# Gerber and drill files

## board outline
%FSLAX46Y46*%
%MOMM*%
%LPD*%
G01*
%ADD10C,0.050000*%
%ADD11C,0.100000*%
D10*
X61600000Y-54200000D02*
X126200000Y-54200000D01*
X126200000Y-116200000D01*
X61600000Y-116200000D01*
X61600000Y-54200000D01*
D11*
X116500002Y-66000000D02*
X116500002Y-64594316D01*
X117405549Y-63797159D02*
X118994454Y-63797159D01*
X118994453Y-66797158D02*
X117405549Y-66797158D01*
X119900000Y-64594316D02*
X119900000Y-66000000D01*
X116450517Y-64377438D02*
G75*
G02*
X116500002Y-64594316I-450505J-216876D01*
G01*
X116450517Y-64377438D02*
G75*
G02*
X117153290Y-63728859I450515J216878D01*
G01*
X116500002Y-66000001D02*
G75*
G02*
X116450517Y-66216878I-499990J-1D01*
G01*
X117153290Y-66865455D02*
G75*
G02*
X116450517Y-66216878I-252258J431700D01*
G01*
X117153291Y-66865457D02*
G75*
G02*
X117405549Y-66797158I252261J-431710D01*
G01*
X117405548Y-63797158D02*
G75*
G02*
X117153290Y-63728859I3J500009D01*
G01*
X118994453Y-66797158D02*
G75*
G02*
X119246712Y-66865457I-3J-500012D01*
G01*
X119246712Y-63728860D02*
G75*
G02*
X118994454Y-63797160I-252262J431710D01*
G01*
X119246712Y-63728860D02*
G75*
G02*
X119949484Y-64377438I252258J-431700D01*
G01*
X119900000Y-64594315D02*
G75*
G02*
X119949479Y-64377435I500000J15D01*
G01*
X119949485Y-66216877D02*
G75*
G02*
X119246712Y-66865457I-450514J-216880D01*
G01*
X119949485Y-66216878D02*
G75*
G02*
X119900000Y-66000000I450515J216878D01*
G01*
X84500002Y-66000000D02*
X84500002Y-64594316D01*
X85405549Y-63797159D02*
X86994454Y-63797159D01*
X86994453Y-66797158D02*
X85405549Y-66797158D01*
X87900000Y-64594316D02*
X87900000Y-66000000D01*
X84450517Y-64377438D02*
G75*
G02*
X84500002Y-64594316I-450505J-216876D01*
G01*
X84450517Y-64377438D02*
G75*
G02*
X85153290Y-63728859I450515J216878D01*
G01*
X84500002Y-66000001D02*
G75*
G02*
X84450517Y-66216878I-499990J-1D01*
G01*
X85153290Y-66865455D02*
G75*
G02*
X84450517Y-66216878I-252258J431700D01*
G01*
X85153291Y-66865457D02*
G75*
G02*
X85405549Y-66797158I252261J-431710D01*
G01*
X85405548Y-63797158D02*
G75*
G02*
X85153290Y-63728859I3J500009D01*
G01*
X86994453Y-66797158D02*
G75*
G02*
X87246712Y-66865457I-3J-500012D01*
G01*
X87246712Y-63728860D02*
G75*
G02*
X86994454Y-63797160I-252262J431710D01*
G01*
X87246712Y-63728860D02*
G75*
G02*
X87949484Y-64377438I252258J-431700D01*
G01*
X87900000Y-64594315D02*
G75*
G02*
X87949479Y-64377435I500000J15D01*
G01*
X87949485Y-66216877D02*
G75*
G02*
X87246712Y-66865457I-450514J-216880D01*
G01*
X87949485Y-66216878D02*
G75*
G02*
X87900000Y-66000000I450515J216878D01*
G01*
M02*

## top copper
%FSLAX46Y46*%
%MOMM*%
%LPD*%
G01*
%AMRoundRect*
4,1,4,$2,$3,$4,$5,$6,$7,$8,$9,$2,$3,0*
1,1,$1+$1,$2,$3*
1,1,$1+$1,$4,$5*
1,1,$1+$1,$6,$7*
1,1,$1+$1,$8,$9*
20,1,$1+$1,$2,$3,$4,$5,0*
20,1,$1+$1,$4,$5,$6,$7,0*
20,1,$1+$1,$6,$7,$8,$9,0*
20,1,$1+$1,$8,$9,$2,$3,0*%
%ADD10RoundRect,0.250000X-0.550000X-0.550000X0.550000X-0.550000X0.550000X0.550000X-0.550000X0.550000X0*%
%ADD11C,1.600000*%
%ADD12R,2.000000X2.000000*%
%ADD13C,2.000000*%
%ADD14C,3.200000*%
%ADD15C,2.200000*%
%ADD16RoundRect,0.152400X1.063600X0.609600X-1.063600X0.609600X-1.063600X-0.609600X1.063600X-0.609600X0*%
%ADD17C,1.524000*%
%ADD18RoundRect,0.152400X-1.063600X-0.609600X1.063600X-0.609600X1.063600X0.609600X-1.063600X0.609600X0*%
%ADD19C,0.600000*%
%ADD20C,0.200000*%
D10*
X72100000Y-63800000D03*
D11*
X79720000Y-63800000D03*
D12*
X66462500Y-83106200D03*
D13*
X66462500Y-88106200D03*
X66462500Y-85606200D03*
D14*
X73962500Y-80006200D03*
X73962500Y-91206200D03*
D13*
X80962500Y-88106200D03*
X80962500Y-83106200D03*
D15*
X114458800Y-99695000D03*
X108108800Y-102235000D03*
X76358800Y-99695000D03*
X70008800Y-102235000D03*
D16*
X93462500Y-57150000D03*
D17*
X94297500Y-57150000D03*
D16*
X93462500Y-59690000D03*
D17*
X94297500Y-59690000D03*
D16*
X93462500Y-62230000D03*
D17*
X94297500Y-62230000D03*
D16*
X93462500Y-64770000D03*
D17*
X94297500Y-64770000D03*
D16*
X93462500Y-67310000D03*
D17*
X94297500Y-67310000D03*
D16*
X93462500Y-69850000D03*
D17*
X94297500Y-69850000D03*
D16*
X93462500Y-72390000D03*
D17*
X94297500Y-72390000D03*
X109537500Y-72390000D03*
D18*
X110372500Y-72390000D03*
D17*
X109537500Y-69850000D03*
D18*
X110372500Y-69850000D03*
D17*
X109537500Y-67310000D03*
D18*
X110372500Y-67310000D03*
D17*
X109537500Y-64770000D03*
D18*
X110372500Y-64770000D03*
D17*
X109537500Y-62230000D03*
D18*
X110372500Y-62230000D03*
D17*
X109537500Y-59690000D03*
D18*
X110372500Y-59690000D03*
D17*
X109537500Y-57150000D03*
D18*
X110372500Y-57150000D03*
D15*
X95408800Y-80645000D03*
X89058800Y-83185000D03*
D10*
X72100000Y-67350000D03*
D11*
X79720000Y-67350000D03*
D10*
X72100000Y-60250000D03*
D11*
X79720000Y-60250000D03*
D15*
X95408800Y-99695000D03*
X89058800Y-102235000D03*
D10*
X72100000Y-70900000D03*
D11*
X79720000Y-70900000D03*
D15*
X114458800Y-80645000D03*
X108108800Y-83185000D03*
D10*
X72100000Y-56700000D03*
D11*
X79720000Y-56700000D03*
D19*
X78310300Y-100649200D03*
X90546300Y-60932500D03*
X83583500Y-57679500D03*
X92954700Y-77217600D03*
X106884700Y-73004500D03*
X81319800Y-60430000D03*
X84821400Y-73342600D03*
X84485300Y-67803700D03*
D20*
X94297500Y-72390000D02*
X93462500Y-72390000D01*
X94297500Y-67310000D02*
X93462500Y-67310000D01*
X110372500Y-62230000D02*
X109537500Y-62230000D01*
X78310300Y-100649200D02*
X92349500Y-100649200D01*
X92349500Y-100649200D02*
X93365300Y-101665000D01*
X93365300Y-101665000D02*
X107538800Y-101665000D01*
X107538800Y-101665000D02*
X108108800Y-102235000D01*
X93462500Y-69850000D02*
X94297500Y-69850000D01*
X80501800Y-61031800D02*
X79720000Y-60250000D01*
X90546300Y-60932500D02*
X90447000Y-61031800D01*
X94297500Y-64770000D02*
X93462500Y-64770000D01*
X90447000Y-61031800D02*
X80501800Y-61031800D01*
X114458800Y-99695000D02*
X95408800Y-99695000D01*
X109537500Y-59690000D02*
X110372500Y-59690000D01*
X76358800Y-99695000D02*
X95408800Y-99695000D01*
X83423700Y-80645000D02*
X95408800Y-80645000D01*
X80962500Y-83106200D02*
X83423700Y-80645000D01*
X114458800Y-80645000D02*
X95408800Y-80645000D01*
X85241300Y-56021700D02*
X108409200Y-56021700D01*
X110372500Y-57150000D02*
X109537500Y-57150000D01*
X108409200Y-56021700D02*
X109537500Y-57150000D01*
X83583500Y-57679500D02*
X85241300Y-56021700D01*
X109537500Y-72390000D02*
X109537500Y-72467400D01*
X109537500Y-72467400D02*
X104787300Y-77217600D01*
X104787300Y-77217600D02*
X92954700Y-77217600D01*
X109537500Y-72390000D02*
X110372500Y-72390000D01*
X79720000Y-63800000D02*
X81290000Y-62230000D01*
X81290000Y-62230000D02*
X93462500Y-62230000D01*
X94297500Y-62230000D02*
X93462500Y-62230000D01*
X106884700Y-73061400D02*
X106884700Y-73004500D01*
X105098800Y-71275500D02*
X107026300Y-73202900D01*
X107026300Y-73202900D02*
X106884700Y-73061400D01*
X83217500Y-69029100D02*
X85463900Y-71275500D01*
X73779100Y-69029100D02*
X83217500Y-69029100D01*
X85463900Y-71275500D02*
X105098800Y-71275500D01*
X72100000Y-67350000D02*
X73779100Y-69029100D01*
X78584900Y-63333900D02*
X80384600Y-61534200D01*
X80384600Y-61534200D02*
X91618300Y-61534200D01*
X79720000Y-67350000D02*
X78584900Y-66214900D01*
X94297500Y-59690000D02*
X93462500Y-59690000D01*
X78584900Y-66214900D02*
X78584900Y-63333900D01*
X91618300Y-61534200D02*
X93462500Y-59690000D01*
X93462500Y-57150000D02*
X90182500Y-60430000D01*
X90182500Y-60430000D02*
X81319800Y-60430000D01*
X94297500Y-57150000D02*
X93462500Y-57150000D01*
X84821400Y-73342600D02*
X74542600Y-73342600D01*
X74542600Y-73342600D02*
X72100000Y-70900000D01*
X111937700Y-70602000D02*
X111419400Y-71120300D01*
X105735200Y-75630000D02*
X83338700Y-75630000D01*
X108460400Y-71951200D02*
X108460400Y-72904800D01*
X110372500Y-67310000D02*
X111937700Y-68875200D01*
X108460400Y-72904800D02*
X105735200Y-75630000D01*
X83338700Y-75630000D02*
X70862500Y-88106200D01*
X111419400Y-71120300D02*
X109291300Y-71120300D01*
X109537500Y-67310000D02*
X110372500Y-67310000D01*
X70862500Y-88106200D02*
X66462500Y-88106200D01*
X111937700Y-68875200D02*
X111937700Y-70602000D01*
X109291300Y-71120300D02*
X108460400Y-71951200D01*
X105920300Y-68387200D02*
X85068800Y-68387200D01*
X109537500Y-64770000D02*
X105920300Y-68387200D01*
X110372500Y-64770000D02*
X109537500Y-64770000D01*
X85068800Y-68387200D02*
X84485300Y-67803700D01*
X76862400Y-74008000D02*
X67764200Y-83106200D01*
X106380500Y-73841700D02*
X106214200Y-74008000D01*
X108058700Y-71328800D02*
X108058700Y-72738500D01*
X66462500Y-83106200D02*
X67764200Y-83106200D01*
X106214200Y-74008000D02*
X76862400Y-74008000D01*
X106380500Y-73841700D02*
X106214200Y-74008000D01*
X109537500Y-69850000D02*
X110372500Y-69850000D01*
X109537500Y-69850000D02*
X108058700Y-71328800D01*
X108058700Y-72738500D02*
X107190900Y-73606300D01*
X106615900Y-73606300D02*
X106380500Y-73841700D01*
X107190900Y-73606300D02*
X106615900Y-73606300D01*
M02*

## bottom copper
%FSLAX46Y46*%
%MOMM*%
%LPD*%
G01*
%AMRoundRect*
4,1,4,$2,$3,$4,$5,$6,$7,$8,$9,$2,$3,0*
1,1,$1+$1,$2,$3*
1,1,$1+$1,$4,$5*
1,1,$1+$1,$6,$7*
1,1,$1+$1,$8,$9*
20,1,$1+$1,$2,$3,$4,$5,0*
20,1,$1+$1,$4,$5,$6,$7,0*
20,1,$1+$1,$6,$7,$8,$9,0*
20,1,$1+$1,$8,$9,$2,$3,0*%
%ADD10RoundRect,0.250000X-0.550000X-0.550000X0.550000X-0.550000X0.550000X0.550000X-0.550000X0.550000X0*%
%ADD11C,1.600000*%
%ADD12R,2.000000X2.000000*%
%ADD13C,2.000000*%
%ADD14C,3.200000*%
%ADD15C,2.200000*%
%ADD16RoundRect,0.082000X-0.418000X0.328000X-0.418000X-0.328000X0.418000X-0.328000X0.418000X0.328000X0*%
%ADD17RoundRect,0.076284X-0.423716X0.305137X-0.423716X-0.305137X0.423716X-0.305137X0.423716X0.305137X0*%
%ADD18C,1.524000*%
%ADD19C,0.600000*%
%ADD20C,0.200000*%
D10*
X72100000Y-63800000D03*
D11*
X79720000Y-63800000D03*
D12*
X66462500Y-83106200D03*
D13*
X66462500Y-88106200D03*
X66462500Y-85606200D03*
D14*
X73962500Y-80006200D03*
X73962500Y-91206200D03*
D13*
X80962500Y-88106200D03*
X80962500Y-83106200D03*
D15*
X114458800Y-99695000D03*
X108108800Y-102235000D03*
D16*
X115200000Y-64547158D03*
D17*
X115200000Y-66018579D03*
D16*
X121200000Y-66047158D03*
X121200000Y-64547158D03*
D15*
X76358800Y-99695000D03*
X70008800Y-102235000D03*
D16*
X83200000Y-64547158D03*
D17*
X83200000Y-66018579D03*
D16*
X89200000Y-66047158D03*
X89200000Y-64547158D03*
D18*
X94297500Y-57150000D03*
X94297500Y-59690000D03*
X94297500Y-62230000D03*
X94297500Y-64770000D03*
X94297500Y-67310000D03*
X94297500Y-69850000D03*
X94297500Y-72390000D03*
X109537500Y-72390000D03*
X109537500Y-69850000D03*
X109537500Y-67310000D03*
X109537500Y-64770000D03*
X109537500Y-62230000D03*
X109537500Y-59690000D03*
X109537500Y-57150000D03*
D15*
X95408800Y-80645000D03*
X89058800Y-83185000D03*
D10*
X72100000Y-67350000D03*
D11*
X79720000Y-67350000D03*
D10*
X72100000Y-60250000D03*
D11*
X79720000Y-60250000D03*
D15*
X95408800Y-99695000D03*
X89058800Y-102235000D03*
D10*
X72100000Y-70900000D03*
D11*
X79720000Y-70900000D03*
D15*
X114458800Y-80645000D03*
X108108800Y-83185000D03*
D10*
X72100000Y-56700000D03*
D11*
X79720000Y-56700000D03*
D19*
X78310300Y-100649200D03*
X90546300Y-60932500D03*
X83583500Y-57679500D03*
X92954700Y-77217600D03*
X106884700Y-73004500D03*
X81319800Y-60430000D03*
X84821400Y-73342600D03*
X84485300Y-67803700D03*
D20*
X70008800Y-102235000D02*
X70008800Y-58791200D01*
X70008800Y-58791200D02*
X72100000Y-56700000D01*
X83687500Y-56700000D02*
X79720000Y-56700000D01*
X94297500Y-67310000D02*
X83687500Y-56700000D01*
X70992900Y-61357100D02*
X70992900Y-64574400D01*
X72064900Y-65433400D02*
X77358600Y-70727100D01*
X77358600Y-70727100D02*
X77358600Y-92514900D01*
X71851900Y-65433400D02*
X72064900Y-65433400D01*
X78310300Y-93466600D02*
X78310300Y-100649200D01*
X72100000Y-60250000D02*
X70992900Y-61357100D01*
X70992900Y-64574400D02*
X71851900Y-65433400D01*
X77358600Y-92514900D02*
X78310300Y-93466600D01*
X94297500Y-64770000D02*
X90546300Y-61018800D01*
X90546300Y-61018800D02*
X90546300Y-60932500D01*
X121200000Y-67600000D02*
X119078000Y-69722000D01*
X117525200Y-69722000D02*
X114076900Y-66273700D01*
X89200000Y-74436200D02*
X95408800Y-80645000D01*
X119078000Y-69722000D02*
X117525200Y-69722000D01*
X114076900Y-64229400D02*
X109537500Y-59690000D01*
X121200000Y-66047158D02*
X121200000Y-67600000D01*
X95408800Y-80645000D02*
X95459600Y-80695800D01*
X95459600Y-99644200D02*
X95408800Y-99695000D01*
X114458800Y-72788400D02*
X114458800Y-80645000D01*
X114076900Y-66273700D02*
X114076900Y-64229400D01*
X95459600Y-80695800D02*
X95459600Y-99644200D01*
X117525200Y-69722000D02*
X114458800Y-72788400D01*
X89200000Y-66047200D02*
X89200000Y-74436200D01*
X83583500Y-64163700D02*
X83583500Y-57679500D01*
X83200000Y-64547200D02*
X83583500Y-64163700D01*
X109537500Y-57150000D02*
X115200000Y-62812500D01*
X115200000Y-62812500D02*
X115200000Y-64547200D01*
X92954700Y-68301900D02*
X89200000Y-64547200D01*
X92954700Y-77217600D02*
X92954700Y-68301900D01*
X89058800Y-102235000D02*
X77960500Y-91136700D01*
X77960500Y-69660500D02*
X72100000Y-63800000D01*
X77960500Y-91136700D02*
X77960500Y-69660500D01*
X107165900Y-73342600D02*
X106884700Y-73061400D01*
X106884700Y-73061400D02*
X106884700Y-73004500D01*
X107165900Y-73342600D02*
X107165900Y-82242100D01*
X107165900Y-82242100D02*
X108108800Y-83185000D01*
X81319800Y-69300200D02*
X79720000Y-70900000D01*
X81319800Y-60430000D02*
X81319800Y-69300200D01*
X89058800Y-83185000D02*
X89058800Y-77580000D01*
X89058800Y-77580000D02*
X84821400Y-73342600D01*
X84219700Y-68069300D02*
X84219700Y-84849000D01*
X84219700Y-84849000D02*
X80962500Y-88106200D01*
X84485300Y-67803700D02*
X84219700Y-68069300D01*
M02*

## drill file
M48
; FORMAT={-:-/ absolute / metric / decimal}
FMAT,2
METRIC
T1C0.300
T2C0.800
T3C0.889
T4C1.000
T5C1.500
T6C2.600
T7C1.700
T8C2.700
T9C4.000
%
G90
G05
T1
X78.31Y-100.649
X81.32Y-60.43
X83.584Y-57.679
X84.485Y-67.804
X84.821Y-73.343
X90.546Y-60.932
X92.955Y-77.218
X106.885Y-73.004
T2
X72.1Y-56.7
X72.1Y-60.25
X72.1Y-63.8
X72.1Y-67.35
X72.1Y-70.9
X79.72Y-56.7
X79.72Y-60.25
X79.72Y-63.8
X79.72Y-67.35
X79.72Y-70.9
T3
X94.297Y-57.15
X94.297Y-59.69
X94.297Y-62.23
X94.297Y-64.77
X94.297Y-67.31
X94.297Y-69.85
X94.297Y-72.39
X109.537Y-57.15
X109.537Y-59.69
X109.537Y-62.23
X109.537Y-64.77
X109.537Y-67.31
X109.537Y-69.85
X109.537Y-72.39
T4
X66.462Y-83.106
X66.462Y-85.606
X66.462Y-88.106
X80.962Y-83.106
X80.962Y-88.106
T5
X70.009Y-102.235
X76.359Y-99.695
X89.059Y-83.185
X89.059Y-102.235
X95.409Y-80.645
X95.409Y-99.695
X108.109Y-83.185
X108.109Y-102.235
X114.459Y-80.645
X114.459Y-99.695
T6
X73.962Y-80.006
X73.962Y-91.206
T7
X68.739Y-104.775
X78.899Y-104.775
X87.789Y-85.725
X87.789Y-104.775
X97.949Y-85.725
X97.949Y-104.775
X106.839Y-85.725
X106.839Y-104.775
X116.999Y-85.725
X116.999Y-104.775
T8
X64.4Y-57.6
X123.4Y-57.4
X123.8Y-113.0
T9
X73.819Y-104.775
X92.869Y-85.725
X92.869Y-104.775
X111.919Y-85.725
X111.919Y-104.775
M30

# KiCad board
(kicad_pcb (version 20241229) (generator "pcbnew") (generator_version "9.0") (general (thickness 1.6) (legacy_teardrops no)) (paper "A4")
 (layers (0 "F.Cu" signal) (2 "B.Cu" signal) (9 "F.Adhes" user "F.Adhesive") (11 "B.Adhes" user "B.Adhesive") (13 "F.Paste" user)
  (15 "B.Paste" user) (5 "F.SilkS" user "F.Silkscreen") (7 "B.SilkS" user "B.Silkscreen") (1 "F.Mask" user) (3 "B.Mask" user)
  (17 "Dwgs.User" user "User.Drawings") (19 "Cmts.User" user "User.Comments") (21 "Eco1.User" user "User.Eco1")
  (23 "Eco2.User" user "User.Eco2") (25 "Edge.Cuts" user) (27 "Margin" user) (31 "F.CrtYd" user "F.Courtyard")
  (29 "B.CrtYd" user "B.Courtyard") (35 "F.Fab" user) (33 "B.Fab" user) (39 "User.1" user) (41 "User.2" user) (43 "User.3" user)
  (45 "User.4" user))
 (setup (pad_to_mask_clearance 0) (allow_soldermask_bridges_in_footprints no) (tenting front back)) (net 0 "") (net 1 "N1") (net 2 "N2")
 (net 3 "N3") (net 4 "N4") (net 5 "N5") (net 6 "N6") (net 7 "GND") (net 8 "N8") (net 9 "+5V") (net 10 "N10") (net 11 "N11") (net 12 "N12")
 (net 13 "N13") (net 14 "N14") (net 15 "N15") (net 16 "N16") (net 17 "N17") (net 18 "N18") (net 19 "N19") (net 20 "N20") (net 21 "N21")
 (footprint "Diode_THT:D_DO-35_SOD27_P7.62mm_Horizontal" (layer "F.Cu") (at 72.1 63.8)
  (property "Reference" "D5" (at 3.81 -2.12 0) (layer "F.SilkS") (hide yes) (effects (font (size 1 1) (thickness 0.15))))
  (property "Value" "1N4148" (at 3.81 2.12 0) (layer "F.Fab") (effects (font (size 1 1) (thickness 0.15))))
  (pad "1" thru_hole roundrect (at 0 0) (size 1.6 1.6) (drill 0.8) (layers "*.Cu" "*.Mask") (remove_unused_layers no)
   (roundrect_rratio 0.15625) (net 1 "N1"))
  (pad "2" thru_hole circle (at 7.62 0) (size 1.6 1.6) (drill 0.8) (layers "*.Cu" "*.Mask") (remove_unused_layers no) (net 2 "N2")))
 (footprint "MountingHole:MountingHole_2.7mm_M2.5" (layer "F.Cu") (at 123.4 57.4)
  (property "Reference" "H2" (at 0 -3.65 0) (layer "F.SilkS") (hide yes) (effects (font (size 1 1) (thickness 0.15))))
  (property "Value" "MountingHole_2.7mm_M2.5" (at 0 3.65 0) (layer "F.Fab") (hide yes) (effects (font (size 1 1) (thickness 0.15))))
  (pad "" np_thru_hole circle (at 0 0) (size 2.7 2.7) (drill 2.7) (layers "*.Cu" "*.Mask")))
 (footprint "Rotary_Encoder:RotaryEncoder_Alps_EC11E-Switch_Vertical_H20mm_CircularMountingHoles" (layer "F.Cu") (at 66.4625 83.1062)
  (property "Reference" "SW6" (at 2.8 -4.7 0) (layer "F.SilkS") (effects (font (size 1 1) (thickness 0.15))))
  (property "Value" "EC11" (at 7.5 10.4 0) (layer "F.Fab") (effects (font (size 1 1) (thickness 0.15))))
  (pad "A" thru_hole rect (at 0 0) (size 2 2) (drill 1) (layers "*.Cu" "*.Mask") (remove_unused_layers no) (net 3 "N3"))
  (pad "B" thru_hole circle (at 0 5) (size 2 2) (drill 1) (layers "*.Cu" "*.Mask") (remove_unused_layers no) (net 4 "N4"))
  (pad "C" thru_hole circle (at 0 2.5) (size 2 2) (drill 1) (layers "*.Cu" "*.Mask") (remove_unused_layers no) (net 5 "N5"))
  (pad "MP" thru_hole circle (at 7.5 -3.1) (size 3.2 3.2) (drill 2.6) (layers "*.Cu" "*.Mask") (remove_unused_layers no))
  (pad "MP" thru_hole circle (at 7.5 8.1) (size 3.2 3.2) (drill 2.6) (layers "*.Cu" "*.Mask") (remove_unused_layers no))
  (pad "S1" thru_hole circle (at 14.5 5) (size 2 2) (drill 1) (layers "*.Cu" "*.Mask") (remove_unused_layers no) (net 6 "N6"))
  (pad "S2" thru_hole circle (at 14.5 0) (size 2 2) (drill 1) (layers "*.Cu" "*.Mask") (remove_unused_layers no) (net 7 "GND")))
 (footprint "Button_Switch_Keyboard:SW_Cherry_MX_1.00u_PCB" (layer "F.Cu") (at 114.4588 99.695)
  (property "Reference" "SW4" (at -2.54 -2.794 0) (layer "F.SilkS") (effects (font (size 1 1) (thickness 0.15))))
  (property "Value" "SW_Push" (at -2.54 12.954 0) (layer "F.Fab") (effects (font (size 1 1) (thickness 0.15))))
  (pad "" np_thru_hole circle (at -7.62 5.08) (size 1.7 1.7) (drill 1.7) (layers "*.Cu" "*.Mask"))
  (pad "" np_thru_hole circle (at -2.54 5.08) (size 4 4) (drill 4) (layers "*.Cu" "*.Mask"))
  (pad "" np_thru_hole circle (at 2.54 5.08) (size 1.7 1.7) (drill 1.7) (layers "*.Cu" "*.Mask"))
  (pad "1" thru_hole circle (at 0 0) (size 2.2 2.2) (drill 1.5) (layers "*.Cu" "*.Mask") (remove_unused_layers no) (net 7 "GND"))
  (pad "2" thru_hole circle (at -6.35 2.54) (size 2.2 2.2) (drill 1.5) (layers "*.Cu" "*.Mask") (remove_unused_layers no) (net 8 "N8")))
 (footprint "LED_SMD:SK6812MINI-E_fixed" (layer "F.Cu") (at 118.2 65.4)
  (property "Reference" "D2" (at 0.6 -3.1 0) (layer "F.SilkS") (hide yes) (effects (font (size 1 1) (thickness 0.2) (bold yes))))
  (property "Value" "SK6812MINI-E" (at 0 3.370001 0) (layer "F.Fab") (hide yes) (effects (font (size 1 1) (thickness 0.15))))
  (fp_line (start -1.699998 0.6) (end -1.699998 -0.805684) (stroke (width 0.1) (type solid)) (layer "Edge.Cuts"))
  (fp_line (start -0.794451 -1.602841) (end 0.794454 -1.602841) (stroke (width 0.1) (type solid)) (layer "Edge.Cuts"))
  (fp_line (start 0.794453 1.397158) (end -0.794451 1.397158) (stroke (width 0.1) (type solid)) (layer "Edge.Cuts"))
  (fp_line (start 1.7 -0.805684) (end 1.7 0.6) (stroke (width 0.1) (type solid)) (layer "Edge.Cuts"))
  (fp_arc (start -1.749483 -1.022562) (mid -1.712526 -0.91691) (end -1.699998 -0.805684) (stroke (width 0.1) (type solid))
   (layer "Edge.Cuts"))
  (fp_arc (start -1.749483 -1.022562) (mid -1.63807 -1.606877) (end -1.04671 -1.671141) (stroke (width 0.1) (type solid))
   (layer "Edge.Cuts"))
  (fp_arc (start -1.699998 0.600001) (mid -1.712526 0.711226) (end -1.749483 0.816878) (stroke (width 0.1) (type solid)) (layer "Edge.Cuts"))
  (fp_arc (start -1.04671 1.465455) (mid -1.638069 1.401192) (end -1.749483 0.816878) (stroke (width 0.1) (type solid)) (layer "Edge.Cuts"))
  (fp_arc (start -1.046709 1.465457) (mid -0.925121 1.414535) (end -0.794451 1.397158) (stroke (width 0.1) (type solid)) (layer "Edge.Cuts"))
  (fp_arc (start -0.794452 -1.602842) (mid -0.925122 -1.620219) (end -1.04671 -1.671141) (stroke (width 0.1) (type solid))
   (layer "Edge.Cuts"))
  (fp_arc (start 0.794453 1.397158) (mid 0.925124 1.414535) (end 1.046712 1.465457) (stroke (width 0.1) (type solid)) (layer "Edge.Cuts"))
  (fp_arc (start 1.046712 -1.67114) (mid 0.925124 -1.620218) (end 0.794454 -1.602841) (stroke (width 0.1) (type solid)) (layer "Edge.Cuts"))
  (fp_arc (start 1.046712 -1.67114) (mid 1.638072 -1.606876) (end 1.749485 -1.022562) (stroke (width 0.1) (type solid)) (layer "Edge.Cuts"))
  (fp_arc (start 1.7 -0.805685) (mid 1.712528 -0.91691) (end 1.749485 -1.022562) (stroke (width 0.1) (type solid)) (layer "Edge.Cuts"))
  (fp_arc (start 1.749485 0.816877) (mid 1.638073 1.401193) (end 1.046712 1.465457) (stroke (width 0.1) (type solid)) (layer "Edge.Cuts"))
  (fp_arc (start 1.749485 0.816878) (mid 1.712528 0.711226) (end 1.7 0.6) (stroke (width 0.1) (type solid)) (layer "Edge.Cuts"))
  (pad "1" smd roundrect (at -3 -0.852842 270) (size 0.82 1) (layers "B.Cu" "B.Mask" "B.Paste") (roundrect_rratio 0.1) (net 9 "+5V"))
  (pad "2" smd roundrect (at -3 0.618579 270) (size 0.762842 1) (layers "B.Cu" "B.Mask" "B.Paste") (roundrect_rratio 0.1))
  (pad "3" smd roundrect (at 3 0.647158 270) (size 0.82 1) (layers "B.Cu" "B.Mask" "B.Paste") (roundrect_rratio 0.1) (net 7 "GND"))
  (pad "4" smd roundrect (at 3 -0.852842 270) (size 0.82 1) (layers "B.Cu" "B.Mask" "B.Paste") (roundrect_rratio 0.1) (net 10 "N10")))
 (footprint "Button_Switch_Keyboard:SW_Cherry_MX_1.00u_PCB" (layer "F.Cu") (at 76.3588 99.695)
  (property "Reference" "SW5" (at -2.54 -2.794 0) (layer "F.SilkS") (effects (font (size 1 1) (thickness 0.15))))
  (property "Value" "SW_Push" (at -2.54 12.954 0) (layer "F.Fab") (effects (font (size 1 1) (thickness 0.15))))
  (pad "" np_thru_hole circle (at -7.62 5.08) (size 1.7 1.7) (drill 1.7) (layers "*.Cu" "*.Mask"))
  (pad "" np_thru_hole circle (at -2.54 5.08) (size 4 4) (drill 4) (layers "*.Cu" "*.Mask"))
  (pad "" np_thru_hole circle (at 2.54 5.08) (size 1.7 1.7) (drill 1.7) (layers "*.Cu" "*.Mask"))
  (pad "1" thru_hole circle (at 0 0) (size 2.2 2.2) (drill 1.5) (layers "*.Cu" "*.Mask") (remove_unused_layers no) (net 7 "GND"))
  (pad "2" thru_hole circle (at -6.35 2.54) (size 2.2 2.2) (drill 1.5) (layers "*.Cu" "*.Mask") (remove_unused_layers no) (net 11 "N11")))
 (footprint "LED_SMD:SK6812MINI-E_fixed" (layer "F.Cu") (at 86.2 65.4)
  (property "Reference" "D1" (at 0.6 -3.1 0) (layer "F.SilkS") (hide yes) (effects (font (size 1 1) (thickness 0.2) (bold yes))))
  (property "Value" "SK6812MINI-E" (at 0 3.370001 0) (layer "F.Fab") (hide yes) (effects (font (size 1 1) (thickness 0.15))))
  (fp_line (start -1.699998 0.6) (end -1.699998 -0.805684) (stroke (width 0.1) (type solid)) (layer "Edge.Cuts"))
  (fp_line (start -0.794451 -1.602841) (end 0.794454 -1.602841) (stroke (width 0.1) (type solid)) (layer "Edge.Cuts"))
  (fp_line (start 0.794453 1.397158) (end -0.794451 1.397158) (stroke (width 0.1) (type solid)) (layer "Edge.Cuts"))
  (fp_line (start 1.7 -0.805684) (end 1.7 0.6) (stroke (width 0.1) (type solid)) (layer "Edge.Cuts"))
  (fp_arc (start -1.749483 -1.022562) (mid -1.712526 -0.91691) (end -1.699998 -0.805684) (stroke (width 0.1) (type solid))
   (layer "Edge.Cuts"))
  (fp_arc (start -1.749483 -1.022562) (mid -1.63807 -1.606877) (end -1.04671 -1.671141) (stroke (width 0.1) (type solid))
   (layer "Edge.Cuts"))
  (fp_arc (start -1.699998 0.600001) (mid -1.712526 0.711226) (end -1.749483 0.816878) (stroke (width 0.1) (type solid)) (layer "Edge.Cuts"))
  (fp_arc (start -1.04671 1.465455) (mid -1.638069 1.401192) (end -1.749483 0.816878) (stroke (width 0.1) (type solid)) (layer "Edge.Cuts"))
  (fp_arc (start -1.046709 1.465457) (mid -0.925121 1.414535) (end -0.794451 1.397158) (stroke (width 0.1) (type solid)) (layer "Edge.Cuts"))
  (fp_arc (start -0.794452 -1.602842) (mid -0.925122 -1.620219) (end -1.04671 -1.671141) (stroke (width 0.1) (type solid))
   (layer "Edge.Cuts"))
  (fp_arc (start 0.794453 1.397158) (mid 0.925124 1.414535) (end 1.046712 1.465457) (stroke (width 0.1) (type solid)) (layer "Edge.Cuts"))
  (fp_arc (start 1.046712 -1.67114) (mid 0.925124 -1.620218) (end 0.794454 -1.602841) (stroke (width 0.1) (type solid)) (layer "Edge.Cuts"))
  (fp_arc (start 1.046712 -1.67114) (mid 1.638072 -1.606876) (end 1.749485 -1.022562) (stroke (width 0.1) (type solid)) (layer "Edge.Cuts"))
  (fp_arc (start 1.7 -0.805685) (mid 1.712528 -0.91691) (end 1.749485 -1.022562) (stroke (width 0.1) (type solid)) (layer "Edge.Cuts"))
  (fp_arc (start 1.749485 0.816877) (mid 1.638073 1.401193) (end 1.046712 1.465457) (stroke (width 0.1) (type solid)) (layer "Edge.Cuts"))
  (fp_arc (start 1.749485 0.816878) (mid 1.712528 0.711226) (end 1.7 0.6) (stroke (width 0.1) (type solid)) (layer "Edge.Cuts"))
  (pad "1" smd roundrect (at -3 -0.852842 270) (size 0.82 1) (layers "B.Cu" "B.Mask" "B.Paste") (roundrect_rratio 0.1) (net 9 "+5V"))
  (pad "2" smd roundrect (at -3 0.618579 270) (size 0.762842 1) (layers "B.Cu" "B.Mask" "B.Paste") (roundrect_rratio 0.1))
  (pad "3" smd roundrect (at 3 0.647158 270) (size 0.82 1) (layers "B.Cu" "B.Mask" "B.Paste") (roundrect_rratio 0.1) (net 7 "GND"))
  (pad "4" smd roundrect (at 3 -0.852842 270) (size 0.82 1) (layers "B.Cu" "B.Mask" "B.Paste") (roundrect_rratio 0.1) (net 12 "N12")))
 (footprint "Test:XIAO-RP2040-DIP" (layer "F.Cu") (at 101.9175 64.77)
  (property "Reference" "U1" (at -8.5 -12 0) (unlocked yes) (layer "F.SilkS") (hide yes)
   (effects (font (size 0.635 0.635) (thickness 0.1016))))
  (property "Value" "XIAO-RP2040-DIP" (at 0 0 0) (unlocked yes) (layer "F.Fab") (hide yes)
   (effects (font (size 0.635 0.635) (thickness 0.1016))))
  (pad "1" smd roundrect (at -8.455 -7.62 180) (size 2.432 1.524) (layers "F.Cu" "F.Mask") (roundrect_rratio 0.1) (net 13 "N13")
   (thermal_bridge_angle 45))
  (pad "1" thru_hole circle (at -7.62 -7.62 180) (size 1.524 1.524) (drill 0.889) (layers "*.Cu" "*.Mask") (remove_unused_layers no)
   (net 13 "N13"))
  (pad "2" smd roundrect (at -8.455 -5.08 180) (size 2.432 1.524) (layers "F.Cu" "F.Mask") (roundrect_rratio 0.1) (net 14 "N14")
   (thermal_bridge_angle 45))
  (pad "2" thru_hole circle (at -7.62 -5.08 180) (size 1.524 1.524) (drill 0.889) (layers "*.Cu" "*.Mask") (remove_unused_layers no)
   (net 14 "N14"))
  (pad "3" smd roundrect (at -8.455 -2.54 180) (size 2.432 1.524) (layers "F.Cu" "F.Mask") (roundrect_rratio 0.1) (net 2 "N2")
   (thermal_bridge_angle 45))
  (pad "3" thru_hole circle (at -7.62 -2.54 180) (size 1.524 1.524) (drill 0.889) (layers "*.Cu" "*.Mask") (remove_unused_layers no)
   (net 2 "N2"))
  (pad "4" smd roundrect (at -8.455 0 180) (size 2.432 1.524) (layers "F.Cu" "F.Mask") (roundrect_rratio 0.1) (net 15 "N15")
   (thermal_bridge_angle 45))
  (pad "4" thru_hole circle (at -7.62 0 180) (size 1.524 1.524) (drill 0.889) (layers "*.Cu" "*.Mask") (remove_unused_layers no)
   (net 15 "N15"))
  (pad "5" smd roundrect (at -8.455 2.54 180) (size 2.432 1.524) (layers "F.Cu" "F.Mask") (roundrect_rratio 0.1) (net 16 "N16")
   (thermal_bridge_angle 45))
  (pad "5" thru_hole circle (at -7.62 2.54 180) (size 1.524 1.524) (drill 0.889) (layers "*.Cu" "*.Mask") (remove_unused_layers no)
   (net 16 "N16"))
  (pad "6" smd roundrect (at -8.455 5.08 180) (size 2.432 1.524) (layers "F.Cu" "F.Mask") (roundrect_rratio 0.1) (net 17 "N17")
   (thermal_bridge_angle 45))
  (pad "6" thru_hole circle (at -7.62 5.08 180) (size 1.524 1.524) (drill 0.889) (layers "*.Cu" "*.Mask") (remove_unused_layers no)
   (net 17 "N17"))
  (pad "7" smd roundrect (at -8.455 7.62 180) (size 2.432 1.524) (layers "F.Cu" "F.Mask") (roundrect_rratio 0.1) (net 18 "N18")
   (thermal_bridge_angle 45))
  (pad "7" thru_hole circle (at -7.62 7.62 180) (size 1.524 1.524) (drill 0.889) (layers "*.Cu" "*.Mask") (remove_unused_layers no)
   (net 18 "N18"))
  (pad "8" thru_hole circle (at 7.62 7.62) (size 1.524 1.524) (drill 0.889) (layers "*.Cu" "*.Mask") (remove_unused_layers no)
   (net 12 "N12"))
  (pad "8" smd roundrect (at 8.455 7.62) (size 2.432 1.524) (layers "F.Cu" "F.Mask") (roundrect_rratio 0.1) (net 12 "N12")
   (thermal_bridge_angle 45))
  (pad "9" thru_hole circle (at 7.62 5.08) (size 1.524 1.524) (drill 0.889) (layers "*.Cu" "*.Mask") (remove_unused_layers no) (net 3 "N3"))
  (pad "9" smd roundrect (at 8.455 5.08) (size 2.432 1.524) (layers "F.Cu" "F.Mask") (roundrect_rratio 0.1) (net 3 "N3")
   (thermal_bridge_angle 45))
  (pad "10" thru_hole circle (at 7.62 2.54) (size 1.524 1.524) (drill 0.889) (layers "*.Cu" "*.Mask") (remove_unused_layers no) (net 4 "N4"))
  (pad "10" smd roundrect (at 8.455 2.54) (size 2.432 1.524) (layers "F.Cu" "F.Mask") (roundrect_rratio 0.1) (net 4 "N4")
   (thermal_bridge_angle 45))
  (pad "11" thru_hole circle (at 7.62 0) (size 1.524 1.524) (drill 0.889) (layers "*.Cu" "*.Mask") (remove_unused_layers no) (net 6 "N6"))
  (pad "11" smd roundrect (at 8.455 0) (size 2.432 1.524) (layers "F.Cu" "F.Mask") (roundrect_rratio 0.1) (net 6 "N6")
   (thermal_bridge_angle 45))
  (pad "12" thru_hole circle (at 7.62 -2.54) (size 1.524 1.524) (drill 0.889) (layers "*.Cu" "*.Mask") (remove_unused_layers no)
   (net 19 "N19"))
  (pad "12" smd roundrect (at 8.455 -2.54) (size 2.432 1.524) (layers "F.Cu" "F.Mask") (roundrect_rratio 0.1) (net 19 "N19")
   (thermal_bridge_angle 45))
  (pad "13" thru_hole circle (at 7.62 -5.08) (size 1.524 1.524) (drill 0.889) (layers "*.Cu" "*.Mask") (remove_unused_layers no)
   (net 7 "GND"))
  (pad "13" smd roundrect (at 8.455 -5.08) (size 2.432 1.524) (layers "F.Cu" "F.Mask") (roundrect_rratio 0.1) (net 7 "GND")
   (thermal_bridge_angle 45))
  (pad "14" thru_hole circle (at 7.62 -7.62) (size 1.524 1.524) (drill 0.889) (layers "*.Cu" "*.Mask") (remove_unused_layers no)
   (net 9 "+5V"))
  (pad "14" smd roundrect (at 8.455 -7.62) (size 2.432 1.524) (layers "F.Cu" "F.Mask") (roundrect_rratio 0.1) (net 9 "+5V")
   (thermal_bridge_angle 45)))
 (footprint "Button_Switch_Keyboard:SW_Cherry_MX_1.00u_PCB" (layer "F.Cu") (at 95.4088 80.645)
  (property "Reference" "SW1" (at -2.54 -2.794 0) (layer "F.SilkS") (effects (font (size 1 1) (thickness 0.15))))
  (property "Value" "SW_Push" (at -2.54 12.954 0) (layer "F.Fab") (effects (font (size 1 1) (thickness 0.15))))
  (pad "" np_thru_hole circle (at -7.62 5.08) (size 1.7 1.7) (drill 1.7) (layers "*.Cu" "*.Mask"))
  (pad "" np_thru_hole circle (at -2.54 5.08) (size 4 4) (drill 4) (layers "*.Cu" "*.Mask"))
  (pad "" np_thru_hole circle (at 2.54 5.08) (size 1.7 1.7) (drill 1.7) (layers "*.Cu" "*.Mask"))
  (pad "1" thru_hole circle (at 0 0) (size 2.2 2.2) (drill 1.5) (layers "*.Cu" "*.Mask") (remove_unused_layers no) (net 7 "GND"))
  (pad "2" thru_hole circle (at -6.35 2.54) (size 2.2 2.2) (drill 1.5) (layers "*.Cu" "*.Mask") (remove_unused_layers no) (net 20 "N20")))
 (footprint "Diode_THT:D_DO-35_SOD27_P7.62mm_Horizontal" (layer "F.Cu") (at 72.1 67.35)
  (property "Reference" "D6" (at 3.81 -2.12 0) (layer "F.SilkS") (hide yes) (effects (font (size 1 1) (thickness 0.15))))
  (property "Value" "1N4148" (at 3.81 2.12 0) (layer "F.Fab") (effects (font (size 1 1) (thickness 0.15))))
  (pad "1" thru_hole roundrect (at 0 0) (size 1.6 1.6) (drill 0.8) (layers "*.Cu" "*.Mask") (remove_unused_layers no)
   (roundrect_rratio 0.15625) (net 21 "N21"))
  (pad "2" thru_hole circle (at 7.62 0) (size 1.6 1.6) (drill 0.8) (layers "*.Cu" "*.Mask") (remove_unused_layers no) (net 14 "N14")))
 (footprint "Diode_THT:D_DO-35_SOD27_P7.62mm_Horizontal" (layer "F.Cu") (at 72.1 60.25)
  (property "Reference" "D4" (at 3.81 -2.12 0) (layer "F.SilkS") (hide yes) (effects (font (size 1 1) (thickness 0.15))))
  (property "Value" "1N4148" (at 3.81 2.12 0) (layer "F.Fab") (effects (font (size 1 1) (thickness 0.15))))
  (pad "1" thru_hole roundrect (at 0 0) (size 1.6 1.6) (drill 0.8) (layers "*.Cu" "*.Mask") (remove_unused_layers no)
   (roundrect_rratio 0.15625) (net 8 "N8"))
  (pad "2" thru_hole circle (at 7.62 0) (size 1.6 1.6) (drill 0.8) (layers "*.Cu" "*.Mask") (remove_unused_layers no) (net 15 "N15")))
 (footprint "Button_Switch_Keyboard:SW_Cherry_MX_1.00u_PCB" (layer "F.Cu") (at 95.4088 99.695)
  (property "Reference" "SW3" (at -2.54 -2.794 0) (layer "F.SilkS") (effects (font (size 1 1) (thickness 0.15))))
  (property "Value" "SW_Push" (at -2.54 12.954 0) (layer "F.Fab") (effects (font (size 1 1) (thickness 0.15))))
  (pad "" np_thru_hole circle (at -7.62 5.08) (size 1.7 1.7) (drill 1.7) (layers "*.Cu" "*.Mask"))
  (pad "" np_thru_hole circle (at -2.54 5.08) (size 4 4) (drill 4) (layers "*.Cu" "*.Mask"))
  (pad "" np_thru_hole circle (at 2.54 5.08) (size 1.7 1.7) (drill 1.7) (layers "*.Cu" "*.Mask"))
  (pad "1" thru_hole circle (at 0 0) (size 2.2 2.2) (drill 1.5) (layers "*.Cu" "*.Mask") (remove_unused_layers no) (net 7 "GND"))
  (pad "2" thru_hole circle (at -6.35 2.54) (size 2.2 2.2) (drill 1.5) (layers "*.Cu" "*.Mask") (remove_unused_layers no) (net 1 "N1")))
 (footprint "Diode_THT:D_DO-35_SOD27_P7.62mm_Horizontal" (layer "F.Cu") (at 72.1 70.9)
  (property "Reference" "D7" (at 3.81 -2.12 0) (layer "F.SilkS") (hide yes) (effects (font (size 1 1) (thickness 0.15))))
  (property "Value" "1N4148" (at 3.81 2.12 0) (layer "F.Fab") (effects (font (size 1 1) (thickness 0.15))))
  (pad "1" thru_hole roundrect (at 0 0) (size 1.6 1.6) (drill 0.8) (layers "*.Cu" "*.Mask") (remove_unused_layers no)
   (roundrect_rratio 0.15625) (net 20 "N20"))
  (pad "2" thru_hole circle (at 7.62 0) (size 1.6 1.6) (drill 0.8) (layers "*.Cu" "*.Mask") (remove_unused_layers no) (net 13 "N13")))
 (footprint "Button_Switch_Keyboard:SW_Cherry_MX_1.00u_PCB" (layer "F.Cu") (at 114.4588 80.645)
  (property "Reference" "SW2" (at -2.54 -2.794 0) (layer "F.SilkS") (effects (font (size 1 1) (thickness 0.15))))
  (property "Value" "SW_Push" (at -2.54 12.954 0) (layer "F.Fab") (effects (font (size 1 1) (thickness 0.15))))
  (pad "" np_thru_hole circle (at -7.62 5.08) (size 1.7 1.7) (drill 1.7) (layers "*.Cu" "*.Mask"))
  (pad "" np_thru_hole circle (at -2.54 5.08) (size 4 4) (drill 4) (layers "*.Cu" "*.Mask"))
  (pad "" np_thru_hole circle (at 2.54 5.08) (size 1.7 1.7) (drill 1.7) (layers "*.Cu" "*.Mask"))
  (pad "1" thru_hole circle (at 0 0) (size 2.2 2.2) (drill 1.5) (layers "*.Cu" "*.Mask") (remove_unused_layers no) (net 7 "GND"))
  (pad "2" thru_hole circle (at -6.35 2.54) (size 2.2 2.2) (drill 1.5) (layers "*.Cu" "*.Mask") (remove_unused_layers no) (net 21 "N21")))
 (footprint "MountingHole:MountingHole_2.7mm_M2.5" (layer "F.Cu") (at 64.4 57.6)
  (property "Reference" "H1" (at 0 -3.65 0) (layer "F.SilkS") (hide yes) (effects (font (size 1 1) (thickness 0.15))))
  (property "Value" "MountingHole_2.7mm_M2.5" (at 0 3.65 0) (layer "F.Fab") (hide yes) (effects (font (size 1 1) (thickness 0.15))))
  (pad "" np_thru_hole circle (at 0 0) (size 2.7 2.7) (drill 2.7) (layers "*.Cu" "*.Mask")))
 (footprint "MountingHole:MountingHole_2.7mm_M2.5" (layer "F.Cu") (at 123.8 113)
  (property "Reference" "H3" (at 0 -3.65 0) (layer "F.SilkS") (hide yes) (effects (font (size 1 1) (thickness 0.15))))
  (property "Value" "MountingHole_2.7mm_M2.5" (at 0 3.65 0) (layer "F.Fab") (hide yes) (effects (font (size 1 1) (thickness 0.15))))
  (pad "" np_thru_hole circle (at 0 0) (size 2.7 2.7) (drill 2.7) (layers "*.Cu" "*.Mask")))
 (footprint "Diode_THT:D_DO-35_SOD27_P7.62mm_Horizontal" (layer "F.Cu") (at 72.1 56.7)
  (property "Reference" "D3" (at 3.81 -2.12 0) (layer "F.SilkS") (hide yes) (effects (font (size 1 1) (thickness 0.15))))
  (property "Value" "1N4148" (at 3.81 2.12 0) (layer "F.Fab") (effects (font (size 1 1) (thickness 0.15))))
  (pad "1" thru_hole roundrect (at 0 0) (size 1.6 1.6) (drill 0.8) (layers "*.Cu" "*.Mask") (remove_unused_layers no)
   (roundrect_rratio 0.15625) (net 11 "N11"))
  (pad "2" thru_hole circle (at 7.62 0) (size 1.6 1.6) (drill 0.8) (layers "*.Cu" "*.Mask") (remove_unused_layers no) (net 16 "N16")))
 (gr_rect (start 61.6 54.2) (end 126.2 116.2) (stroke (width 0.05) (type default)) (fill no) (layer "Edge.Cuts"))
 (segment (start 94.2975 72.39) (end 93.4625 72.39) (width 0.2) (layer "F.Cu") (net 18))
 (segment (start 70.0088 102.235) (end 70.0088 58.7912) (width 0.2) (layer "B.Cu") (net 11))
 (segment (start 70.0088 58.7912) (end 72.1 56.7) (width 0.2) (layer "B.Cu") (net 11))
 (segment (start 94.2975 67.31) (end 93.4625 67.31) (width 0.2) (layer "F.Cu") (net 16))
 (segment (start 83.6875 56.7) (end 79.72 56.7) (width 0.2) (layer "B.Cu") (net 16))
 (segment (start 94.2975 67.31) (end 83.6875 56.7) (width 0.2) (layer "B.Cu") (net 16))
 (segment (start 110.3725 62.23) (end 109.5375 62.23) (width 0.2) (layer "F.Cu") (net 19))
 (segment (start 78.3103 100.6492) (end 92.3495 100.6492) (width 0.2) (layer "F.Cu") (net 8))
 (segment (start 92.3495 100.6492) (end 93.3653 101.665) (width 0.2) (layer "F.Cu") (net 8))
 (segment (start 93.3653 101.665) (end 107.5388 101.665) (width 0.2) (layer "F.Cu") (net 8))
 (segment (start 107.5388 101.665) (end 108.1088 102.235) (width 0.2) (layer "F.Cu") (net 8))
 (via (at 78.3103 100.6492) (size 0.6) (drill 0.3) (layers "F.Cu" "B.Cu") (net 8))
 (segment (start 70.9929 61.3571) (end 70.9929 64.5744) (width 0.2) (layer "B.Cu") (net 8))
 (segment (start 72.0649 65.4334) (end 77.3586 70.7271) (width 0.2) (layer "B.Cu") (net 8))
 (segment (start 77.3586 70.7271) (end 77.3586 92.5149) (width 0.2) (layer "B.Cu") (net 8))
 (segment (start 71.8519 65.4334) (end 72.0649 65.4334) (width 0.2) (layer "B.Cu") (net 8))
 (segment (start 78.3103 93.4666) (end 78.3103 100.6492) (width 0.2) (layer "B.Cu") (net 8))
 (segment (start 72.1 60.25) (end 70.9929 61.3571) (width 0.2) (layer "B.Cu") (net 8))
 (segment (start 70.9929 64.5744) (end 71.8519 65.4334) (width 0.2) (layer "B.Cu") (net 8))
 (segment (start 77.3586 92.5149) (end 78.3103 93.4666) (width 0.2) (layer "B.Cu") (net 8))
 (segment (start 93.4625 69.85) (end 94.2975 69.85) (width 0.2) (layer "F.Cu") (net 17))
 (segment (start 80.5018 61.0318) (end 79.72 60.25) (width 0.2) (layer "F.Cu") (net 15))
 (segment (start 90.5463 60.9325) (end 90.447 61.0318) (width 0.2) (layer "F.Cu") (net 15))
 (segment (start 94.2975 64.77) (end 93.4625 64.77) (width 0.2) (layer "F.Cu") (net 15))
 (segment (start 90.447 61.0318) (end 80.5018 61.0318) (width 0.2) (layer "F.Cu") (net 15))
 (via (at 90.5463 60.9325) (size 0.6) (drill 0.3) (layers "F.Cu" "B.Cu") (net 15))
 (segment (start 94.2975 64.77) (end 90.5463 61.0188) (width 0.2) (layer "B.Cu") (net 15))
 (segment (start 90.5463 61.0188) (end 90.5463 60.9325) (width 0.2) (layer "B.Cu") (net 15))
 (segment (start 114.4588 99.695) (end 95.4088 99.695) (width 0.2) (layer "F.Cu") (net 7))
 (segment (start 109.5375 59.69) (end 110.3725 59.69) (width 0.2) (layer "F.Cu") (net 7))
 (segment (start 76.3588 99.695) (end 95.4088 99.695) (width 0.2) (layer "F.Cu") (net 7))
 (segment (start 83.4237 80.645) (end 95.4088 80.645) (width 0.2) (layer "F.Cu") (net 7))
 (segment (start 80.9625 83.1062) (end 83.4237 80.645) (width 0.2) (layer "F.Cu") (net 7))
 (segment (start 114.4588 80.645) (end 95.4088 80.645) (width 0.2) (layer "F.Cu") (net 7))
 (segment (start 121.2 67.6) (end 119.078 69.722) (width 0.2) (layer "B.Cu") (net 7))
 (segment (start 117.5252 69.722) (end 114.0769 66.2737) (width 0.2) (layer "B.Cu") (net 7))
 (segment (start 89.2 74.4362) (end 95.4088 80.645) (width 0.2) (layer "B.Cu") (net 7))
 (segment (start 119.078 69.722) (end 117.5252 69.722) (width 0.2) (layer "B.Cu") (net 7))
 (segment (start 114.0769 64.2294) (end 109.5375 59.69) (width 0.2) (layer "B.Cu") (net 7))
 (segment (start 121.2 66.047158) (end 121.2 67.6) (width 0.2) (layer "B.Cu") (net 7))
 (segment (start 95.4088 80.645) (end 95.4596 80.6958) (width 0.2) (layer "B.Cu") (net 7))
 (segment (start 95.4596 99.6442) (end 95.4088 99.695) (width 0.2) (layer "B.Cu") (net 7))
 (segment (start 114.4588 72.7884) (end 114.4588 80.645) (width 0.2) (layer "B.Cu") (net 7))
 (segment (start 114.0769 66.2737) (end 114.0769 64.2294) (width 0.2) (layer "B.Cu") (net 7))
 (segment (start 95.4596 80.6958) (end 95.4596 99.6442) (width 0.2) (layer "B.Cu") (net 7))
 (segment (start 117.5252 69.722) (end 114.4588 72.7884) (width 0.2) (layer "B.Cu") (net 7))
 (segment (start 89.2 66.0472) (end 89.2 74.4362) (width 0.2) (layer "B.Cu") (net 7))
 (segment (start 85.2413 56.0217) (end 108.4092 56.0217) (width 0.2) (layer "F.Cu") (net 9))
 (segment (start 110.3725 57.15) (end 109.5375 57.15) (width 0.2) (layer "F.Cu") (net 9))
 (segment (start 108.4092 56.0217) (end 109.5375 57.15) (width 0.2) (layer "F.Cu") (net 9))
 (segment (start 83.5835 57.6795) (end 85.2413 56.0217) (width 0.2) (layer "F.Cu") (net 9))
 (via (at 83.5835 57.6795) (size 0.6) (drill 0.3) (layers "F.Cu" "B.Cu") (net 9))
 (segment (start 83.5835 64.1637) (end 83.5835 57.6795) (width 0.2) (layer "B.Cu") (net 9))
 (segment (start 83.2 64.5472) (end 83.5835 64.1637) (width 0.2) (layer "B.Cu") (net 9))
 (segment (start 109.5375 57.15) (end 115.2 62.8125) (width 0.2) (layer "B.Cu") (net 9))
 (segment (start 115.2 62.8125) (end 115.2 64.5472) (width 0.2) (layer "B.Cu") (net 9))
 (segment (start 109.5375 72.39) (end 109.5375 72.4674) (width 0.2) (layer "F.Cu") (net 12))
 (segment (start 109.5375 72.4674) (end 104.7873 77.2176) (width 0.2) (layer "F.Cu") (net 12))
 (segment (start 104.7873 77.2176) (end 92.9547 77.2176) (width 0.2) (layer "F.Cu") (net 12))
 (segment (start 109.5375 72.39) (end 110.3725 72.39) (width 0.2) (layer "F.Cu") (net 12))
 (via (at 92.9547 77.2176) (size 0.6) (drill 0.3) (layers "F.Cu" "B.Cu") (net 12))
 (segment (start 92.9547 68.3019) (end 89.2 64.5472) (width 0.2) (layer "B.Cu") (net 12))
 (segment (start 92.9547 77.2176) (end 92.9547 68.3019) (width 0.2) (layer "B.Cu") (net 12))
 (segment (start 89.0588 102.235) (end 77.9605 91.1367) (width 0.2) (layer "B.Cu") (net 1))
 (segment (start 77.9605 69.6605) (end 72.1 63.8) (width 0.2) (layer "B.Cu") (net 1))
 (segment (start 77.9605 91.1367) (end 77.9605 69.6605) (width 0.2) (layer "B.Cu") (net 1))
 (segment (start 79.72 63.8) (end 81.29 62.23) (width 0.2) (layer "F.Cu") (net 2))
 (segment (start 81.29 62.23) (end 93.4625 62.23) (width 0.2) (layer "F.Cu") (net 2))
 (segment (start 94.2975 62.23) (end 93.4625 62.23) (width 0.2) (layer "F.Cu") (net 2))
 (segment (start 106.8847 73.0614) (end 106.8847 73.0045) (width 0.2) (layer "F.Cu") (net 21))
 (segment (start 105.0988 71.2755) (end 107.0263 73.2029) (width 0.2) (layer "F.Cu") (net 21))
 (segment (start 107.0263 73.2029) (end 106.8847 73.0614) (width 0.2) (layer "F.Cu") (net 21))
 (segment (start 83.2175 69.0291) (end 85.4639 71.2755) (width 0.2) (layer "F.Cu") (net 21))
 (segment (start 73.7791 69.0291) (end 83.2175 69.0291) (width 0.2) (layer "F.Cu") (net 21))
 (segment (start 85.4639 71.2755) (end 105.0988 71.2755) (width 0.2) (layer "F.Cu") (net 21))
 (segment (start 72.1 67.35) (end 73.7791 69.0291) (width 0.2) (layer "F.Cu") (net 21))
 (via (at 106.8847 73.0045) (size 0.6) (drill 0.3) (layers "F.Cu" "B.Cu") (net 21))
 (segment (start 107.1659 73.3426) (end 106.8847 73.0614) (width 0.2) (layer "B.Cu") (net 21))
 (segment (start 106.8847 73.0614) (end 106.8847 73.0045) (width 0.2) (layer "B.Cu") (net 21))
 (segment (start 107.1659 73.3426) (end 107.1659 82.2421) (width 0.2) (layer "B.Cu") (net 21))
 (segment (start 107.1659 82.2421) (end 108.1088 83.185) (width 0.2) (layer "B.Cu") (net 21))
 (segment (start 78.5849 63.3339) (end 80.3846 61.5342) (width 0.2) (layer "F.Cu") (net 14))
 (segment (start 80.3846 61.5342) (end 91.6183 61.5342) (width 0.2) (layer "F.Cu") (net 14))
 (segment (start 79.72 67.35) (end 78.5849 66.2149) (width 0.2) (layer "F.Cu") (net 14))
 (segment (start 94.2975 59.69) (end 93.4625 59.69) (width 0.2) (layer "F.Cu") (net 14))
 (segment (start 78.5849 66.2149) (end 78.5849 63.3339) (width 0.2) (layer "F.Cu") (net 14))
 (segment (start 91.6183 61.5342) (end 93.4625 59.69) (width 0.2) (layer "F.Cu") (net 14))
 (segment (start 93.4625 57.15) (end 90.1825 60.43) (width 0.2) (layer "F.Cu") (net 13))
 (segment (start 90.1825 60.43) (end 81.3198 60.43) (width 0.2) (layer "F.Cu") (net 13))
 (segment (start 94.2975 57.15) (end 93.4625 57.15) (width 0.2) (layer "F.Cu") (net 13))
 (via (at 81.3198 60.43) (size 0.6) (drill 0.3) (layers "F.Cu" "B.Cu") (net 13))
 (segment (start 81.3198 69.3002) (end 79.72 70.9) (width 0.2) (layer "B.Cu") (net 13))
 (segment (start 81.3198 60.43) (end 81.3198 69.3002) (width 0.2) (layer "B.Cu") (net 13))
 (segment (start 84.8214 73.3426) (end 74.5426 73.3426) (width 0.2) (layer "F.Cu") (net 20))
 (segment (start 74.5426 73.3426) (end 72.1 70.9) (width 0.2) (layer "F.Cu") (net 20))
 (via (at 84.8214 73.3426) (size 0.6) (drill 0.3) (layers "F.Cu" "B.Cu") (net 20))
 (segment (start 89.0588 83.185) (end 89.0588 77.58) (width 0.2) (layer "B.Cu") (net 20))
 (segment (start 89.0588 77.58) (end 84.8214 73.3426) (width 0.2) (layer "B.Cu") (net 20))
 (segment (start 111.9377 70.602) (end 111.4194 71.1203) (width 0.2) (layer "F.Cu") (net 4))
 (segment (start 105.7352 75.63) (end 83.3387 75.63) (width 0.2) (layer "F.Cu") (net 4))
 (segment (start 108.4604 71.9512) (end 108.4604 72.9048) (width 0.2) (layer "F.Cu") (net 4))
 (segment (start 110.3725 67.31) (end 111.9377 68.8752) (width 0.2) (layer "F.Cu") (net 4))
 (segment (start 108.4604 72.9048) (end 105.7352 75.63) (width 0.2) (layer "F.Cu") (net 4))
 (segment (start 83.3387 75.63) (end 70.8625 88.1062) (width 0.2) (layer "F.Cu") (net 4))
 (segment (start 111.4194 71.1203) (end 109.2913 71.1203) (width 0.2) (layer "F.Cu") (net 4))
 (segment (start 109.5375 67.31) (end 110.3725 67.31) (width 0.2) (layer "F.Cu") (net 4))
 (segment (start 70.8625 88.1062) (end 66.4625 88.1062) (width 0.2) (layer "F.Cu") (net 4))
 (segment (start 111.9377 68.8752) (end 111.9377 70.602) (width 0.2) (layer "F.Cu") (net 4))
 (segment (start 109.2913 71.1203) (end 108.4604 71.9512) (width 0.2) (layer "F.Cu") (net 4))
 (segment (start 105.9203 68.3872) (end 85.0688 68.3872) (width 0.2) (layer "F.Cu") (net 6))
 (segment (start 109.5375 64.77) (end 105.9203 68.3872) (width 0.2) (layer "F.Cu") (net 6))
 (segment (start 110.3725 64.77) (end 109.5375 64.77) (width 0.2) (layer "F.Cu") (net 6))
 (segment (start 85.0688 68.3872) (end 84.4853 67.8037) (width 0.2) (layer "F.Cu") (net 6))
 (via (at 84.4853 67.8037) (size 0.6) (drill 0.3) (layers "F.Cu" "B.Cu") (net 6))
 (segment (start 84.2197 68.0693) (end 84.2197 84.849) (width 0.2) (layer "B.Cu") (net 6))
 (segment (start 84.2197 84.849) (end 80.9625 88.1062) (width 0.2) (layer "B.Cu") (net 6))
 (segment (start 84.4853 67.8037) (end 84.2197 68.0693) (width 0.2) (layer "B.Cu") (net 6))
 (segment (start 76.8624 74.008) (end 67.7642 83.1062) (width 0.2) (layer "F.Cu") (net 3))
 (segment (start 106.3805 73.8417) (end 106.2142 74.008) (width 0.2) (layer "F.Cu") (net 3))
 (segment (start 108.0587 71.3288) (end 108.0587 72.7385) (width 0.2) (layer "F.Cu") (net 3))
 (segment (start 66.4625 83.1062) (end 67.7642 83.1062) (width 0.2) (layer "F.Cu") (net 3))
 (segment (start 106.2142 74.008) (end 76.8624 74.008) (width 0.2) (layer "F.Cu") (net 3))
 (segment (start 106.3805 73.8417) (end 106.2142 74.008) (width 0.2) (layer "F.Cu") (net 3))
 (segment (start 109.5375 69.85) (end 110.3725 69.85) (width 0.2) (layer "F.Cu") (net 3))
 (segment (start 109.5375 69.85) (end 108.0587 71.3288) (width 0.2) (layer "F.Cu") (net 3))
 (segment (start 108.0587 72.7385) (end 107.1909 73.6063) (width 0.2) (layer "F.Cu") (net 3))
 (segment (start 106.6159 73.6063) (end 106.3805 73.8417) (width 0.2) (layer "F.Cu") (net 3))
 (segment (start 107.1909 73.6063) (end 106.6159 73.6063) (width 0.2) (layer "F.Cu") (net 3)))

